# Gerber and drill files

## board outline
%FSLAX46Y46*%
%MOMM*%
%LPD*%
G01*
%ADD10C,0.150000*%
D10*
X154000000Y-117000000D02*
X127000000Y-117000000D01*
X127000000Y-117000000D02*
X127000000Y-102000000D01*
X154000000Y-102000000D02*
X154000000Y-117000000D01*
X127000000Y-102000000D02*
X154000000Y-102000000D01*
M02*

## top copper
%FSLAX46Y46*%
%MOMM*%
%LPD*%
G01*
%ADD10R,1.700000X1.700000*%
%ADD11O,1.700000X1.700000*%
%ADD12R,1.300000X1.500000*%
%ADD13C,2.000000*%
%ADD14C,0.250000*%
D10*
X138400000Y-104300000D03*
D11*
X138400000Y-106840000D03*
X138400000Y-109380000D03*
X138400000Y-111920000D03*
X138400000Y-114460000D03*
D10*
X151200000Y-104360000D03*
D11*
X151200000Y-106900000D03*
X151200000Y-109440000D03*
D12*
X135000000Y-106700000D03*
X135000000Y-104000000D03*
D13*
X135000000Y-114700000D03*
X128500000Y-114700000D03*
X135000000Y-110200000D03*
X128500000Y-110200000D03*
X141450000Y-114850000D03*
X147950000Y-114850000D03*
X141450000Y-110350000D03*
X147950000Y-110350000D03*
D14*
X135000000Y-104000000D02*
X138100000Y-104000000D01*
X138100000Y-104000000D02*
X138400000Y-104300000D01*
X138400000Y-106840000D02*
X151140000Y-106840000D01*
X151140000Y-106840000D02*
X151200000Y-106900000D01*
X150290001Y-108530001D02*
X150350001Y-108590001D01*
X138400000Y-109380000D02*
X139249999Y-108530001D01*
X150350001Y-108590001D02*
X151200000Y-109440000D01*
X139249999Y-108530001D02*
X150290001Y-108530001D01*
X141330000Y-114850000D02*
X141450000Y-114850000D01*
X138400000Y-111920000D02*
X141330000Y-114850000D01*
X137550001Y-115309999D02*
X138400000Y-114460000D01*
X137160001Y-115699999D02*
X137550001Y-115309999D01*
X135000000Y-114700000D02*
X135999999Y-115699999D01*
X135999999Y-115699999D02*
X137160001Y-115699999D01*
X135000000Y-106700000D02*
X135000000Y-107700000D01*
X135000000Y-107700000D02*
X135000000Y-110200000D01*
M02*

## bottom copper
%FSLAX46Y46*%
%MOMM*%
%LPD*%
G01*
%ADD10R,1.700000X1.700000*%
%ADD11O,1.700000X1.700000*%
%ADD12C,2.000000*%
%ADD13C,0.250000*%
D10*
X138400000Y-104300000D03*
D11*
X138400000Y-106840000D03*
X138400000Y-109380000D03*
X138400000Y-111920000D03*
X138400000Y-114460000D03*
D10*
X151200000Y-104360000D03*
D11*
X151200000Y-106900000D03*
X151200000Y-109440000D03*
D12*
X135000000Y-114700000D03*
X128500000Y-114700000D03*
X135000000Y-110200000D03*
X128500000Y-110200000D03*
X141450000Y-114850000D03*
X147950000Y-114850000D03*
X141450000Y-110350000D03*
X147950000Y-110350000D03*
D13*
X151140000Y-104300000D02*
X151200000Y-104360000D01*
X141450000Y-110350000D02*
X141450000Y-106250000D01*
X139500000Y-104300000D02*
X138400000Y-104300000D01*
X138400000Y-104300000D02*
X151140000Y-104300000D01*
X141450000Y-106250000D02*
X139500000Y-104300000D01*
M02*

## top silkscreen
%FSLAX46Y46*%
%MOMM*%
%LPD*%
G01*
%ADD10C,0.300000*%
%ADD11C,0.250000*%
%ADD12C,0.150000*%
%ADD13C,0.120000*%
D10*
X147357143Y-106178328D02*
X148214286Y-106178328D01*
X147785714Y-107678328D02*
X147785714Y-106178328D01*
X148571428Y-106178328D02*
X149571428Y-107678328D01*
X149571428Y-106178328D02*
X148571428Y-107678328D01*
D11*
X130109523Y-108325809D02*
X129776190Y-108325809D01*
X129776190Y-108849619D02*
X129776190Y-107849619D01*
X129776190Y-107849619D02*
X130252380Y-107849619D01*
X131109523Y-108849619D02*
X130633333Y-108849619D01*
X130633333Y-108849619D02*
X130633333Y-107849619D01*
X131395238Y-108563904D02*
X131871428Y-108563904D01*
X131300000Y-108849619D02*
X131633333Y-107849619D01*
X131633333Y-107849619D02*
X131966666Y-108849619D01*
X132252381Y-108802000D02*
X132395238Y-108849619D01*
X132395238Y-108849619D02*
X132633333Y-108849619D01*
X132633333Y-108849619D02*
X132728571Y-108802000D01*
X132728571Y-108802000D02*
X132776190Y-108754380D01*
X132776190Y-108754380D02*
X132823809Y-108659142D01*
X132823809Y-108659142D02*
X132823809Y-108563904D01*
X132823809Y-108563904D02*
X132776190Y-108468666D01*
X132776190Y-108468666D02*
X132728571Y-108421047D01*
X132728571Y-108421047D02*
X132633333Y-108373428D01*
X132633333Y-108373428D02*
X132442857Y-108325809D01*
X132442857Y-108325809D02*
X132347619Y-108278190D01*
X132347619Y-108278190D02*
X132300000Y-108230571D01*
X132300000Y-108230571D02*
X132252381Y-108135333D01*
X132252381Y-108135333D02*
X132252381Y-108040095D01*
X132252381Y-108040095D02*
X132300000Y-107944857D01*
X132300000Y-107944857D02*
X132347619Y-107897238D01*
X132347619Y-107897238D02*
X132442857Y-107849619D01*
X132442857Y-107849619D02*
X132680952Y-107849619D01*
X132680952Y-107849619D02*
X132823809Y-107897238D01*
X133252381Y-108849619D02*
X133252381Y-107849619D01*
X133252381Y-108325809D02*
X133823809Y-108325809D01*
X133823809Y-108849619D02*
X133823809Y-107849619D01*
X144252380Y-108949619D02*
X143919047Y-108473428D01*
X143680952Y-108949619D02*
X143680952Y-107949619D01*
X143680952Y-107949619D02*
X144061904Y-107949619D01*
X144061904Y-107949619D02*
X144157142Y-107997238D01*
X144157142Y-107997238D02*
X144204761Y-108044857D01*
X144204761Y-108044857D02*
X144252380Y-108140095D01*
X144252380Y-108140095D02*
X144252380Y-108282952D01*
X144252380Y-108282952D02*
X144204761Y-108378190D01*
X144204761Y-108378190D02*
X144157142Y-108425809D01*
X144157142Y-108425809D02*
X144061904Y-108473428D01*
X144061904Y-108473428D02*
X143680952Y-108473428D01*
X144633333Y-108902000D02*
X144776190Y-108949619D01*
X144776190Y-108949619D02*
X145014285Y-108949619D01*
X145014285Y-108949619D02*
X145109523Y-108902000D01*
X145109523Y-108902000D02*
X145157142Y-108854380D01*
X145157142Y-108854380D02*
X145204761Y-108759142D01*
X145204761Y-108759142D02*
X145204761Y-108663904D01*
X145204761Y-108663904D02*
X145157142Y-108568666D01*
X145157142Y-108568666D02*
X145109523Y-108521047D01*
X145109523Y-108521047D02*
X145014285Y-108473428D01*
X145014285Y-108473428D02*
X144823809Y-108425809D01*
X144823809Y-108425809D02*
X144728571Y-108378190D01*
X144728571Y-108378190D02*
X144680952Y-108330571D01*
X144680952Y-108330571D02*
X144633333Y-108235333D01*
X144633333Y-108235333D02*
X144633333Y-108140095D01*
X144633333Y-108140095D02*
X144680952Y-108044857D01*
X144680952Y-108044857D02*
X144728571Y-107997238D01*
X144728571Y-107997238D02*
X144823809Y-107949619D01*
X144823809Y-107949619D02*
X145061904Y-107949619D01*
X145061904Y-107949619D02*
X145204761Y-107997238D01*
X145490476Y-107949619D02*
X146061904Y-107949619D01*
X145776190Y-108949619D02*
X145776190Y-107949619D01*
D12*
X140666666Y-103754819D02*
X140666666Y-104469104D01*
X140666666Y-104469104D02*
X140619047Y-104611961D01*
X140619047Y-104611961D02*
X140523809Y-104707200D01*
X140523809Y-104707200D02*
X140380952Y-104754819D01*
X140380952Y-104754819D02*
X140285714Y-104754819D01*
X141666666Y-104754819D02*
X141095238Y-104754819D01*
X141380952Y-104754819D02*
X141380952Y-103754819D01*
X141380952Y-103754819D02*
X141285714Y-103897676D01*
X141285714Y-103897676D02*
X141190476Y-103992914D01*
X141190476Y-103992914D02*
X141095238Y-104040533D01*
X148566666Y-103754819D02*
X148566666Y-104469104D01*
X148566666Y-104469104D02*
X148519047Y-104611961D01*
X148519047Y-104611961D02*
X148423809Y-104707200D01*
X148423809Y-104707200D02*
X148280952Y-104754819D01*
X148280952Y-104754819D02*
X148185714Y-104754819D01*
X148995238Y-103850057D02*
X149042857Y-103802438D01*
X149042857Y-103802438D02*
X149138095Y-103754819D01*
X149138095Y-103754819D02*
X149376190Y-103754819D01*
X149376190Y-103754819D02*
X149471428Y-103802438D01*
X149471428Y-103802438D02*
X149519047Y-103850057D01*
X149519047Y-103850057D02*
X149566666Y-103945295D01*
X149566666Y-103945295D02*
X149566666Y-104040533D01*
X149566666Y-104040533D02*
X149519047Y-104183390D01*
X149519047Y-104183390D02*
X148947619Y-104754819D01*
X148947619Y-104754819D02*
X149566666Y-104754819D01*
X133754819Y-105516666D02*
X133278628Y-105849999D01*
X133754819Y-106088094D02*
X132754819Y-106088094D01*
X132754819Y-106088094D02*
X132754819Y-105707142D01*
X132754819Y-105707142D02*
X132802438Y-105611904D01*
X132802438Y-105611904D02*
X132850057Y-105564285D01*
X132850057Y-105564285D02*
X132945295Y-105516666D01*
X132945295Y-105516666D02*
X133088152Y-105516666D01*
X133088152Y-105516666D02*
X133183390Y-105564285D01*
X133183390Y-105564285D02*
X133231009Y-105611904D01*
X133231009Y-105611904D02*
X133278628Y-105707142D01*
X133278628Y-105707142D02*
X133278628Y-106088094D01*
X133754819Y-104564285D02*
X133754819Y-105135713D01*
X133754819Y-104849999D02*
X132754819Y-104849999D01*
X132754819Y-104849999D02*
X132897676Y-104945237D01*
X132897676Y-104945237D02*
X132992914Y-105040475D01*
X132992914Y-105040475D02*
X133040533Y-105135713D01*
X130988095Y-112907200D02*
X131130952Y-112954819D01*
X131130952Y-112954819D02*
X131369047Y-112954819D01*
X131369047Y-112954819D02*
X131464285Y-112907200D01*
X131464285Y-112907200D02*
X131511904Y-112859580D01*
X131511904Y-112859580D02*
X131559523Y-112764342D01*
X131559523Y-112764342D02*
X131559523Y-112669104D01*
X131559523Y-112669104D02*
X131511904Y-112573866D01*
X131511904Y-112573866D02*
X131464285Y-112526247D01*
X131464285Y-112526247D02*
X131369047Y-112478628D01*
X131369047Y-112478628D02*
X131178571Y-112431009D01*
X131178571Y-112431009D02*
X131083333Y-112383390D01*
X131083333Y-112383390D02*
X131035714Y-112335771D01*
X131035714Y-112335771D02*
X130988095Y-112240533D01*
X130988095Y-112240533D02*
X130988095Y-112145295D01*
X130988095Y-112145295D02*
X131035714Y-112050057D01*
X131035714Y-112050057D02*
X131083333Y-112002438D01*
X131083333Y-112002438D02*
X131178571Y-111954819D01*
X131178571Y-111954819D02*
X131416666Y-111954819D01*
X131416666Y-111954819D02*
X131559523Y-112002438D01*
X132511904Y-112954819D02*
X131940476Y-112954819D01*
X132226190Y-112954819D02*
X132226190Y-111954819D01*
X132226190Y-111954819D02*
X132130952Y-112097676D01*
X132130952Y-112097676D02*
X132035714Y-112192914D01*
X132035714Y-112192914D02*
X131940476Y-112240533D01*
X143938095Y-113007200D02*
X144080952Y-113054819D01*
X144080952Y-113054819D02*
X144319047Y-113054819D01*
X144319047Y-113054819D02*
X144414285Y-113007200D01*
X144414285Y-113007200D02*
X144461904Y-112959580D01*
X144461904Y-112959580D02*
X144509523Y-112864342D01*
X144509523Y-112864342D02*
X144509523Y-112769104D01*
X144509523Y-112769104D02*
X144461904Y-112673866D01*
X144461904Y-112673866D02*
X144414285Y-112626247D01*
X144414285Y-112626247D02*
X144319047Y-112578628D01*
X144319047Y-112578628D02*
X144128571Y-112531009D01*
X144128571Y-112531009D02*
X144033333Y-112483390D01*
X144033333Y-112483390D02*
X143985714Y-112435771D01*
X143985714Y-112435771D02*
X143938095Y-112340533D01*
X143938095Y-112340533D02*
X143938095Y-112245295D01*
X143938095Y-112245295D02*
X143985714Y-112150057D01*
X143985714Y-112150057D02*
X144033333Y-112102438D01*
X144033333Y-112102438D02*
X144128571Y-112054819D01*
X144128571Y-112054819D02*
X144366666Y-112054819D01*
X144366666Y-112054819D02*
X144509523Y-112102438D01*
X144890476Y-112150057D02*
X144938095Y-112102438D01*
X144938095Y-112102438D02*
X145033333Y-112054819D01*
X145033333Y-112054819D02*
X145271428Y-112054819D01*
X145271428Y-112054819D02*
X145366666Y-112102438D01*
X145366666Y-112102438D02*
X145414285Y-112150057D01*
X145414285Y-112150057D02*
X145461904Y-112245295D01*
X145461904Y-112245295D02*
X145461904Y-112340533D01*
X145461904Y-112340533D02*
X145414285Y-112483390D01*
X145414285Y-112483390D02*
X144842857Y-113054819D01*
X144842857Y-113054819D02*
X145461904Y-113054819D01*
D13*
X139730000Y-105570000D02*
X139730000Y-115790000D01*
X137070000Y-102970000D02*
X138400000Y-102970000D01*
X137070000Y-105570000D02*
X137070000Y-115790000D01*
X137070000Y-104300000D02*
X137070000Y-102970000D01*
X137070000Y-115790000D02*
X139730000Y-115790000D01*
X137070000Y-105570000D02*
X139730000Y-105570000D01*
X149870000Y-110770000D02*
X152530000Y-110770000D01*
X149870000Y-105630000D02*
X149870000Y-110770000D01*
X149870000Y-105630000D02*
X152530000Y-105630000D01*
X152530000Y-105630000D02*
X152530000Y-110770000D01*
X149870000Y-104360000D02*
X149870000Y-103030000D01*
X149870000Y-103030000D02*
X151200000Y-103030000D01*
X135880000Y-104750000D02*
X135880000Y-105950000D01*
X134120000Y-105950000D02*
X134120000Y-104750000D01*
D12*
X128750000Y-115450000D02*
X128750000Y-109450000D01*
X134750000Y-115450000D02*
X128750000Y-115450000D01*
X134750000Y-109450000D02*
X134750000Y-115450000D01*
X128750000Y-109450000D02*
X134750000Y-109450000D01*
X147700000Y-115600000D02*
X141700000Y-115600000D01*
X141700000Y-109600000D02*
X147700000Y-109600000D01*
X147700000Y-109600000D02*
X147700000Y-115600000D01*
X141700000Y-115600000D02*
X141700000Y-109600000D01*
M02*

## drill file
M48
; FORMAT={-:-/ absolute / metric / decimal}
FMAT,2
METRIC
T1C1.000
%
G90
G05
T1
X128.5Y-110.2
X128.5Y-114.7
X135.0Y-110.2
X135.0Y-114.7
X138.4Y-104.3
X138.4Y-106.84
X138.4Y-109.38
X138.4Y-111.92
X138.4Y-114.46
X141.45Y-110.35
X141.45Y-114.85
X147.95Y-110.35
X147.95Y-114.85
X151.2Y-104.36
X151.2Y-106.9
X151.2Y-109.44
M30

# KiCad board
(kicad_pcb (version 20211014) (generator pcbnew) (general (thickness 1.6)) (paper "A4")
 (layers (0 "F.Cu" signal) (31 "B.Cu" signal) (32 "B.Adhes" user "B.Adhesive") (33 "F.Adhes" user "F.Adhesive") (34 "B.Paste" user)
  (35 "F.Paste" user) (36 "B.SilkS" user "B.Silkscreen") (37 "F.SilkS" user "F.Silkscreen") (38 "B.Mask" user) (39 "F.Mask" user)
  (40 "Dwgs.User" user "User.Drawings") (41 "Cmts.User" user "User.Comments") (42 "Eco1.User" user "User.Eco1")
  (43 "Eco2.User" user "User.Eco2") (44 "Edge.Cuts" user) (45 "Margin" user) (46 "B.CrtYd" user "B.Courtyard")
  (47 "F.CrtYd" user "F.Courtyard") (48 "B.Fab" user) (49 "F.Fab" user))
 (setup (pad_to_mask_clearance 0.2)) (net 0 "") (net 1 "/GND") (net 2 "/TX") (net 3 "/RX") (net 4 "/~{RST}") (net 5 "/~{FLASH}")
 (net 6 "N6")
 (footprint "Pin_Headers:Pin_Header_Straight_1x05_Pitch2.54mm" (layer "F.Cu") (at 138.4 104.3)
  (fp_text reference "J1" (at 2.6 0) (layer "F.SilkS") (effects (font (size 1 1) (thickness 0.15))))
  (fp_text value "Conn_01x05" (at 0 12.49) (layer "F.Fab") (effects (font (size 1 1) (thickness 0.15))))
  (fp_line (start 1.33 1.27) (end 1.33 11.49) (layer "F.SilkS") (width 0.12))
  (fp_line (start -1.33 -1.33) (end 0 -1.33) (layer "F.SilkS") (width 0.12))
  (fp_line (start -1.33 1.27) (end -1.33 11.49) (layer "F.SilkS") (width 0.12))
  (fp_line (start -1.33 0) (end -1.33 -1.33) (layer "F.SilkS") (width 0.12))
  (fp_line (start -1.33 11.49) (end 1.33 11.49) (layer "F.SilkS") (width 0.12))
  (fp_line (start -1.33 1.27) (end 1.33 1.27) (layer "F.SilkS") (width 0.12))
  (pad "1" thru_hole rect locked (at 0 0) (size 1.7 1.7) (drill 1) (layers *.Cu *.Mask) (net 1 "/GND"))
  (pad "2" thru_hole oval locked (at 0 2.54) (size 1.7 1.7) (drill 1) (layers *.Cu *.Mask) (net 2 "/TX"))
  (pad "3" thru_hole oval locked (at 0 5.08) (size 1.7 1.7) (drill 1) (layers *.Cu *.Mask) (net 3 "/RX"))
  (pad "4" thru_hole oval locked (at 0 7.62) (size 1.7 1.7) (drill 1) (layers *.Cu *.Mask) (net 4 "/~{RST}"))
  (pad "5" thru_hole oval locked (at 0 10.16) (size 1.7 1.7) (drill 1) (layers *.Cu *.Mask) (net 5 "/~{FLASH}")))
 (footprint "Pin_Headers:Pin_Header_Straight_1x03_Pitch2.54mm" (layer "F.Cu") (at 151.2 104.36)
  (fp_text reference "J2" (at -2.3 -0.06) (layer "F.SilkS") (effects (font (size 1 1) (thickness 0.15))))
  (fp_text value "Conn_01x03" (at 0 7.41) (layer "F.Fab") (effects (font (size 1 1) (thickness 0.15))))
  (fp_line (start -1.33 6.41) (end 1.33 6.41) (layer "F.SilkS") (width 0.12))
  (fp_line (start -1.33 1.27) (end -1.33 6.41) (layer "F.SilkS") (width 0.12))
  (fp_line (start -1.33 1.27) (end 1.33 1.27) (layer "F.SilkS") (width 0.12))
  (fp_line (start 1.33 1.27) (end 1.33 6.41) (layer "F.SilkS") (width 0.12))
  (fp_line (start -1.33 0) (end -1.33 -1.33) (layer "F.SilkS") (width 0.12))
  (fp_line (start -1.33 -1.33) (end 0 -1.33) (layer "F.SilkS") (width 0.12))
  (pad "1" thru_hole rect locked (at 0 0) (size 1.7 1.7) (drill 1) (layers *.Cu *.Mask) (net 1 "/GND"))
  (pad "2" thru_hole oval locked (at 0 2.54) (size 1.7 1.7) (drill 1) (layers *.Cu *.Mask) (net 2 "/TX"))
  (pad "3" thru_hole oval locked (at 0 5.08) (size 1.7 1.7) (drill 1) (layers *.Cu *.Mask) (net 3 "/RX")))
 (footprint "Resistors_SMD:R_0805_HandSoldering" (layer "F.Cu") (at 135 105.35 90)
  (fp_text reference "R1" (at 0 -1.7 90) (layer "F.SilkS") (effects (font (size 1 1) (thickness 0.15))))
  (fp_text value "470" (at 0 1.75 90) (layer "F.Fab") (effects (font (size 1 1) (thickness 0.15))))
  (fp_line (start 0.6 0.88) (end -0.6 0.88) (layer "F.SilkS") (width 0.12))
  (fp_line (start -0.6 -0.88) (end 0.6 -0.88) (layer "F.SilkS") (width 0.12))
  (pad "1" smd rect locked (at -1.35 0 90) (size 1.5 1.3) (layers "F.Cu" "F.Paste" "F.Mask") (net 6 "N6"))
  (pad "2" smd rect locked (at 1.35 0 90) (size 1.5 1.3) (layers "F.Cu" "F.Paste" "F.Mask") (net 1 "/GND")))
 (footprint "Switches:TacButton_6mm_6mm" (layer "F.Cu") (at 131.75 112.45 180)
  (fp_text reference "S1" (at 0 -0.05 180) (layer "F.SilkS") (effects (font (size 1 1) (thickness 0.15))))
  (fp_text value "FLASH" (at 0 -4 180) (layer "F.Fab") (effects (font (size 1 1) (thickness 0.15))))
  (fp_line (start 3 -3) (end 3 3) (layer "F.SilkS") (width 0.15))
  (fp_line (start -3 -3) (end 3 -3) (layer "F.SilkS") (width 0.15))
  (fp_line (start -3 3) (end -3 -3) (layer "F.SilkS") (width 0.15))
  (fp_line (start 3 3) (end -3 3) (layer "F.SilkS") (width 0.15))
  (pad "1" thru_hole circle locked (at -3.25 -2.25 180) (size 2 2) (drill 1) (layers *.Cu *.Mask) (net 5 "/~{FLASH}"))
  (pad "1" thru_hole circle locked (at 3.25 -2.25 180) (size 2 2) (drill 1) (layers *.Cu *.Mask) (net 5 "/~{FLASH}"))
  (pad "2" thru_hole circle locked (at -3.25 2.25 180) (size 2 2) (drill 1) (layers *.Cu *.Mask) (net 6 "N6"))
  (pad "2" thru_hole circle locked (at 3.25 2.25 180) (size 2 2) (drill 1) (layers *.Cu *.Mask) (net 6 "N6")))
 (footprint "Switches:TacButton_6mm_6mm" (layer "F.Cu") (at 144.7 112.6 180)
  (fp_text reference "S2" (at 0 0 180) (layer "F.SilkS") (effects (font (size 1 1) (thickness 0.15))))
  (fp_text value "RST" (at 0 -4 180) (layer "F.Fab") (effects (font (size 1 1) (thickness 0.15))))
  (fp_line (start -3 -3) (end 3 -3) (layer "F.SilkS") (width 0.15))
  (fp_line (start 3 3) (end -3 3) (layer "F.SilkS") (width 0.15))
  (fp_line (start -3 3) (end -3 -3) (layer "F.SilkS") (width 0.15))
  (fp_line (start 3 -3) (end 3 3) (layer "F.SilkS") (width 0.15))
  (pad "1" thru_hole circle locked (at 3.25 -2.25 180) (size 2 2) (drill 1) (layers *.Cu *.Mask) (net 4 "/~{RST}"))
  (pad "1" thru_hole circle locked (at -3.25 -2.25 180) (size 2 2) (drill 1) (layers *.Cu *.Mask) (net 4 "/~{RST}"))
  (pad "2" thru_hole circle locked (at 3.25 2.25 180) (size 2 2) (drill 1) (layers *.Cu *.Mask) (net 1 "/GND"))
  (pad "2" thru_hole circle locked (at -3.25 2.25 180) (size 2 2) (drill 1) (layers *.Cu *.Mask) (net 1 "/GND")))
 (gr_line (start 154 117) (end 127 117) (layer "Edge.Cuts") (width 0.15))
 (gr_line (start 127 117) (end 127 102) (layer "Edge.Cuts") (width 0.15))
 (gr_line (start 154 102) (end 154 117) (layer "Edge.Cuts") (width 0.15))
 (gr_line (start 127 102) (end 154 102) (layer "Edge.Cuts") (width 0.15))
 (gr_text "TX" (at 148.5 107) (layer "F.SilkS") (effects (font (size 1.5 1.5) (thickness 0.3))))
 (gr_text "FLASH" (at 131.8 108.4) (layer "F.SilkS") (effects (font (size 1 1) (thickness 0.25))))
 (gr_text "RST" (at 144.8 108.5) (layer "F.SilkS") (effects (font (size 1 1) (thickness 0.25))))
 (segment (start 135 104) (end 138.1 104) (width 0.25) (layer "F.Cu") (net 1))
 (segment (start 138.1 104) (end 138.4 104.3) (width 0.25) (layer "F.Cu") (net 1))
 (segment (start 151.14 104.3) (end 151.2 104.36) (width 0.25) (layer "B.Cu") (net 1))
 (segment (start 141.45 110.35) (end 141.45 106.25) (width 0.25) (layer "B.Cu") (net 1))
 (segment (start 139.5 104.3) (end 138.4 104.3) (width 0.25) (layer "B.Cu") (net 1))
 (segment (start 138.4 104.3) (end 151.14 104.3) (width 0.25) (layer "B.Cu") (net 1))
 (segment (start 141.45 106.25) (end 139.5 104.3) (width 0.25) (layer "B.Cu") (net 1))
 (segment (start 138.4 106.84) (end 151.14 106.84) (width 0.25) (layer "F.Cu") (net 2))
 (segment (start 151.14 106.84) (end 151.2 106.9) (width 0.25) (layer "F.Cu") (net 2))
 (segment (start 150.290001 108.530001) (end 150.350001 108.590001) (width 0.25) (layer "F.Cu") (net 3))
 (segment (start 138.4 109.38) (end 139.249999 108.530001) (width 0.25) (layer "F.Cu") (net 3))
 (segment (start 150.350001 108.590001) (end 151.2 109.44) (width 0.25) (layer "F.Cu") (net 3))
 (segment (start 139.249999 108.530001) (end 150.290001 108.530001) (width 0.25) (layer "F.Cu") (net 3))
 (segment (start 141.33 114.85) (end 141.45 114.85) (width 0.25) (layer "F.Cu") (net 4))
 (segment (start 138.4 111.92) (end 141.33 114.85) (width 0.25) (layer "F.Cu") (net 4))
 (segment (start 137.550001 115.309999) (end 138.4 114.46) (width 0.25) (layer "F.Cu") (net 5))
 (segment (start 137.160001 115.699999) (end 137.550001 115.309999) (width 0.25) (layer "F.Cu") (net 5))
 (segment (start 135 114.7) (end 135.999999 115.699999) (width 0.25) (layer "F.Cu") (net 5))
 (segment (start 135.999999 115.699999) (end 137.160001 115.699999) (width 0.25) (layer "F.Cu") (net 5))
 (segment (start 135 106.7) (end 135 107.7) (width 0.25) (layer "F.Cu") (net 6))
 (segment (start 135 107.7) (end 135 110.2) (width 0.25) (layer "F.Cu") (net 6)))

